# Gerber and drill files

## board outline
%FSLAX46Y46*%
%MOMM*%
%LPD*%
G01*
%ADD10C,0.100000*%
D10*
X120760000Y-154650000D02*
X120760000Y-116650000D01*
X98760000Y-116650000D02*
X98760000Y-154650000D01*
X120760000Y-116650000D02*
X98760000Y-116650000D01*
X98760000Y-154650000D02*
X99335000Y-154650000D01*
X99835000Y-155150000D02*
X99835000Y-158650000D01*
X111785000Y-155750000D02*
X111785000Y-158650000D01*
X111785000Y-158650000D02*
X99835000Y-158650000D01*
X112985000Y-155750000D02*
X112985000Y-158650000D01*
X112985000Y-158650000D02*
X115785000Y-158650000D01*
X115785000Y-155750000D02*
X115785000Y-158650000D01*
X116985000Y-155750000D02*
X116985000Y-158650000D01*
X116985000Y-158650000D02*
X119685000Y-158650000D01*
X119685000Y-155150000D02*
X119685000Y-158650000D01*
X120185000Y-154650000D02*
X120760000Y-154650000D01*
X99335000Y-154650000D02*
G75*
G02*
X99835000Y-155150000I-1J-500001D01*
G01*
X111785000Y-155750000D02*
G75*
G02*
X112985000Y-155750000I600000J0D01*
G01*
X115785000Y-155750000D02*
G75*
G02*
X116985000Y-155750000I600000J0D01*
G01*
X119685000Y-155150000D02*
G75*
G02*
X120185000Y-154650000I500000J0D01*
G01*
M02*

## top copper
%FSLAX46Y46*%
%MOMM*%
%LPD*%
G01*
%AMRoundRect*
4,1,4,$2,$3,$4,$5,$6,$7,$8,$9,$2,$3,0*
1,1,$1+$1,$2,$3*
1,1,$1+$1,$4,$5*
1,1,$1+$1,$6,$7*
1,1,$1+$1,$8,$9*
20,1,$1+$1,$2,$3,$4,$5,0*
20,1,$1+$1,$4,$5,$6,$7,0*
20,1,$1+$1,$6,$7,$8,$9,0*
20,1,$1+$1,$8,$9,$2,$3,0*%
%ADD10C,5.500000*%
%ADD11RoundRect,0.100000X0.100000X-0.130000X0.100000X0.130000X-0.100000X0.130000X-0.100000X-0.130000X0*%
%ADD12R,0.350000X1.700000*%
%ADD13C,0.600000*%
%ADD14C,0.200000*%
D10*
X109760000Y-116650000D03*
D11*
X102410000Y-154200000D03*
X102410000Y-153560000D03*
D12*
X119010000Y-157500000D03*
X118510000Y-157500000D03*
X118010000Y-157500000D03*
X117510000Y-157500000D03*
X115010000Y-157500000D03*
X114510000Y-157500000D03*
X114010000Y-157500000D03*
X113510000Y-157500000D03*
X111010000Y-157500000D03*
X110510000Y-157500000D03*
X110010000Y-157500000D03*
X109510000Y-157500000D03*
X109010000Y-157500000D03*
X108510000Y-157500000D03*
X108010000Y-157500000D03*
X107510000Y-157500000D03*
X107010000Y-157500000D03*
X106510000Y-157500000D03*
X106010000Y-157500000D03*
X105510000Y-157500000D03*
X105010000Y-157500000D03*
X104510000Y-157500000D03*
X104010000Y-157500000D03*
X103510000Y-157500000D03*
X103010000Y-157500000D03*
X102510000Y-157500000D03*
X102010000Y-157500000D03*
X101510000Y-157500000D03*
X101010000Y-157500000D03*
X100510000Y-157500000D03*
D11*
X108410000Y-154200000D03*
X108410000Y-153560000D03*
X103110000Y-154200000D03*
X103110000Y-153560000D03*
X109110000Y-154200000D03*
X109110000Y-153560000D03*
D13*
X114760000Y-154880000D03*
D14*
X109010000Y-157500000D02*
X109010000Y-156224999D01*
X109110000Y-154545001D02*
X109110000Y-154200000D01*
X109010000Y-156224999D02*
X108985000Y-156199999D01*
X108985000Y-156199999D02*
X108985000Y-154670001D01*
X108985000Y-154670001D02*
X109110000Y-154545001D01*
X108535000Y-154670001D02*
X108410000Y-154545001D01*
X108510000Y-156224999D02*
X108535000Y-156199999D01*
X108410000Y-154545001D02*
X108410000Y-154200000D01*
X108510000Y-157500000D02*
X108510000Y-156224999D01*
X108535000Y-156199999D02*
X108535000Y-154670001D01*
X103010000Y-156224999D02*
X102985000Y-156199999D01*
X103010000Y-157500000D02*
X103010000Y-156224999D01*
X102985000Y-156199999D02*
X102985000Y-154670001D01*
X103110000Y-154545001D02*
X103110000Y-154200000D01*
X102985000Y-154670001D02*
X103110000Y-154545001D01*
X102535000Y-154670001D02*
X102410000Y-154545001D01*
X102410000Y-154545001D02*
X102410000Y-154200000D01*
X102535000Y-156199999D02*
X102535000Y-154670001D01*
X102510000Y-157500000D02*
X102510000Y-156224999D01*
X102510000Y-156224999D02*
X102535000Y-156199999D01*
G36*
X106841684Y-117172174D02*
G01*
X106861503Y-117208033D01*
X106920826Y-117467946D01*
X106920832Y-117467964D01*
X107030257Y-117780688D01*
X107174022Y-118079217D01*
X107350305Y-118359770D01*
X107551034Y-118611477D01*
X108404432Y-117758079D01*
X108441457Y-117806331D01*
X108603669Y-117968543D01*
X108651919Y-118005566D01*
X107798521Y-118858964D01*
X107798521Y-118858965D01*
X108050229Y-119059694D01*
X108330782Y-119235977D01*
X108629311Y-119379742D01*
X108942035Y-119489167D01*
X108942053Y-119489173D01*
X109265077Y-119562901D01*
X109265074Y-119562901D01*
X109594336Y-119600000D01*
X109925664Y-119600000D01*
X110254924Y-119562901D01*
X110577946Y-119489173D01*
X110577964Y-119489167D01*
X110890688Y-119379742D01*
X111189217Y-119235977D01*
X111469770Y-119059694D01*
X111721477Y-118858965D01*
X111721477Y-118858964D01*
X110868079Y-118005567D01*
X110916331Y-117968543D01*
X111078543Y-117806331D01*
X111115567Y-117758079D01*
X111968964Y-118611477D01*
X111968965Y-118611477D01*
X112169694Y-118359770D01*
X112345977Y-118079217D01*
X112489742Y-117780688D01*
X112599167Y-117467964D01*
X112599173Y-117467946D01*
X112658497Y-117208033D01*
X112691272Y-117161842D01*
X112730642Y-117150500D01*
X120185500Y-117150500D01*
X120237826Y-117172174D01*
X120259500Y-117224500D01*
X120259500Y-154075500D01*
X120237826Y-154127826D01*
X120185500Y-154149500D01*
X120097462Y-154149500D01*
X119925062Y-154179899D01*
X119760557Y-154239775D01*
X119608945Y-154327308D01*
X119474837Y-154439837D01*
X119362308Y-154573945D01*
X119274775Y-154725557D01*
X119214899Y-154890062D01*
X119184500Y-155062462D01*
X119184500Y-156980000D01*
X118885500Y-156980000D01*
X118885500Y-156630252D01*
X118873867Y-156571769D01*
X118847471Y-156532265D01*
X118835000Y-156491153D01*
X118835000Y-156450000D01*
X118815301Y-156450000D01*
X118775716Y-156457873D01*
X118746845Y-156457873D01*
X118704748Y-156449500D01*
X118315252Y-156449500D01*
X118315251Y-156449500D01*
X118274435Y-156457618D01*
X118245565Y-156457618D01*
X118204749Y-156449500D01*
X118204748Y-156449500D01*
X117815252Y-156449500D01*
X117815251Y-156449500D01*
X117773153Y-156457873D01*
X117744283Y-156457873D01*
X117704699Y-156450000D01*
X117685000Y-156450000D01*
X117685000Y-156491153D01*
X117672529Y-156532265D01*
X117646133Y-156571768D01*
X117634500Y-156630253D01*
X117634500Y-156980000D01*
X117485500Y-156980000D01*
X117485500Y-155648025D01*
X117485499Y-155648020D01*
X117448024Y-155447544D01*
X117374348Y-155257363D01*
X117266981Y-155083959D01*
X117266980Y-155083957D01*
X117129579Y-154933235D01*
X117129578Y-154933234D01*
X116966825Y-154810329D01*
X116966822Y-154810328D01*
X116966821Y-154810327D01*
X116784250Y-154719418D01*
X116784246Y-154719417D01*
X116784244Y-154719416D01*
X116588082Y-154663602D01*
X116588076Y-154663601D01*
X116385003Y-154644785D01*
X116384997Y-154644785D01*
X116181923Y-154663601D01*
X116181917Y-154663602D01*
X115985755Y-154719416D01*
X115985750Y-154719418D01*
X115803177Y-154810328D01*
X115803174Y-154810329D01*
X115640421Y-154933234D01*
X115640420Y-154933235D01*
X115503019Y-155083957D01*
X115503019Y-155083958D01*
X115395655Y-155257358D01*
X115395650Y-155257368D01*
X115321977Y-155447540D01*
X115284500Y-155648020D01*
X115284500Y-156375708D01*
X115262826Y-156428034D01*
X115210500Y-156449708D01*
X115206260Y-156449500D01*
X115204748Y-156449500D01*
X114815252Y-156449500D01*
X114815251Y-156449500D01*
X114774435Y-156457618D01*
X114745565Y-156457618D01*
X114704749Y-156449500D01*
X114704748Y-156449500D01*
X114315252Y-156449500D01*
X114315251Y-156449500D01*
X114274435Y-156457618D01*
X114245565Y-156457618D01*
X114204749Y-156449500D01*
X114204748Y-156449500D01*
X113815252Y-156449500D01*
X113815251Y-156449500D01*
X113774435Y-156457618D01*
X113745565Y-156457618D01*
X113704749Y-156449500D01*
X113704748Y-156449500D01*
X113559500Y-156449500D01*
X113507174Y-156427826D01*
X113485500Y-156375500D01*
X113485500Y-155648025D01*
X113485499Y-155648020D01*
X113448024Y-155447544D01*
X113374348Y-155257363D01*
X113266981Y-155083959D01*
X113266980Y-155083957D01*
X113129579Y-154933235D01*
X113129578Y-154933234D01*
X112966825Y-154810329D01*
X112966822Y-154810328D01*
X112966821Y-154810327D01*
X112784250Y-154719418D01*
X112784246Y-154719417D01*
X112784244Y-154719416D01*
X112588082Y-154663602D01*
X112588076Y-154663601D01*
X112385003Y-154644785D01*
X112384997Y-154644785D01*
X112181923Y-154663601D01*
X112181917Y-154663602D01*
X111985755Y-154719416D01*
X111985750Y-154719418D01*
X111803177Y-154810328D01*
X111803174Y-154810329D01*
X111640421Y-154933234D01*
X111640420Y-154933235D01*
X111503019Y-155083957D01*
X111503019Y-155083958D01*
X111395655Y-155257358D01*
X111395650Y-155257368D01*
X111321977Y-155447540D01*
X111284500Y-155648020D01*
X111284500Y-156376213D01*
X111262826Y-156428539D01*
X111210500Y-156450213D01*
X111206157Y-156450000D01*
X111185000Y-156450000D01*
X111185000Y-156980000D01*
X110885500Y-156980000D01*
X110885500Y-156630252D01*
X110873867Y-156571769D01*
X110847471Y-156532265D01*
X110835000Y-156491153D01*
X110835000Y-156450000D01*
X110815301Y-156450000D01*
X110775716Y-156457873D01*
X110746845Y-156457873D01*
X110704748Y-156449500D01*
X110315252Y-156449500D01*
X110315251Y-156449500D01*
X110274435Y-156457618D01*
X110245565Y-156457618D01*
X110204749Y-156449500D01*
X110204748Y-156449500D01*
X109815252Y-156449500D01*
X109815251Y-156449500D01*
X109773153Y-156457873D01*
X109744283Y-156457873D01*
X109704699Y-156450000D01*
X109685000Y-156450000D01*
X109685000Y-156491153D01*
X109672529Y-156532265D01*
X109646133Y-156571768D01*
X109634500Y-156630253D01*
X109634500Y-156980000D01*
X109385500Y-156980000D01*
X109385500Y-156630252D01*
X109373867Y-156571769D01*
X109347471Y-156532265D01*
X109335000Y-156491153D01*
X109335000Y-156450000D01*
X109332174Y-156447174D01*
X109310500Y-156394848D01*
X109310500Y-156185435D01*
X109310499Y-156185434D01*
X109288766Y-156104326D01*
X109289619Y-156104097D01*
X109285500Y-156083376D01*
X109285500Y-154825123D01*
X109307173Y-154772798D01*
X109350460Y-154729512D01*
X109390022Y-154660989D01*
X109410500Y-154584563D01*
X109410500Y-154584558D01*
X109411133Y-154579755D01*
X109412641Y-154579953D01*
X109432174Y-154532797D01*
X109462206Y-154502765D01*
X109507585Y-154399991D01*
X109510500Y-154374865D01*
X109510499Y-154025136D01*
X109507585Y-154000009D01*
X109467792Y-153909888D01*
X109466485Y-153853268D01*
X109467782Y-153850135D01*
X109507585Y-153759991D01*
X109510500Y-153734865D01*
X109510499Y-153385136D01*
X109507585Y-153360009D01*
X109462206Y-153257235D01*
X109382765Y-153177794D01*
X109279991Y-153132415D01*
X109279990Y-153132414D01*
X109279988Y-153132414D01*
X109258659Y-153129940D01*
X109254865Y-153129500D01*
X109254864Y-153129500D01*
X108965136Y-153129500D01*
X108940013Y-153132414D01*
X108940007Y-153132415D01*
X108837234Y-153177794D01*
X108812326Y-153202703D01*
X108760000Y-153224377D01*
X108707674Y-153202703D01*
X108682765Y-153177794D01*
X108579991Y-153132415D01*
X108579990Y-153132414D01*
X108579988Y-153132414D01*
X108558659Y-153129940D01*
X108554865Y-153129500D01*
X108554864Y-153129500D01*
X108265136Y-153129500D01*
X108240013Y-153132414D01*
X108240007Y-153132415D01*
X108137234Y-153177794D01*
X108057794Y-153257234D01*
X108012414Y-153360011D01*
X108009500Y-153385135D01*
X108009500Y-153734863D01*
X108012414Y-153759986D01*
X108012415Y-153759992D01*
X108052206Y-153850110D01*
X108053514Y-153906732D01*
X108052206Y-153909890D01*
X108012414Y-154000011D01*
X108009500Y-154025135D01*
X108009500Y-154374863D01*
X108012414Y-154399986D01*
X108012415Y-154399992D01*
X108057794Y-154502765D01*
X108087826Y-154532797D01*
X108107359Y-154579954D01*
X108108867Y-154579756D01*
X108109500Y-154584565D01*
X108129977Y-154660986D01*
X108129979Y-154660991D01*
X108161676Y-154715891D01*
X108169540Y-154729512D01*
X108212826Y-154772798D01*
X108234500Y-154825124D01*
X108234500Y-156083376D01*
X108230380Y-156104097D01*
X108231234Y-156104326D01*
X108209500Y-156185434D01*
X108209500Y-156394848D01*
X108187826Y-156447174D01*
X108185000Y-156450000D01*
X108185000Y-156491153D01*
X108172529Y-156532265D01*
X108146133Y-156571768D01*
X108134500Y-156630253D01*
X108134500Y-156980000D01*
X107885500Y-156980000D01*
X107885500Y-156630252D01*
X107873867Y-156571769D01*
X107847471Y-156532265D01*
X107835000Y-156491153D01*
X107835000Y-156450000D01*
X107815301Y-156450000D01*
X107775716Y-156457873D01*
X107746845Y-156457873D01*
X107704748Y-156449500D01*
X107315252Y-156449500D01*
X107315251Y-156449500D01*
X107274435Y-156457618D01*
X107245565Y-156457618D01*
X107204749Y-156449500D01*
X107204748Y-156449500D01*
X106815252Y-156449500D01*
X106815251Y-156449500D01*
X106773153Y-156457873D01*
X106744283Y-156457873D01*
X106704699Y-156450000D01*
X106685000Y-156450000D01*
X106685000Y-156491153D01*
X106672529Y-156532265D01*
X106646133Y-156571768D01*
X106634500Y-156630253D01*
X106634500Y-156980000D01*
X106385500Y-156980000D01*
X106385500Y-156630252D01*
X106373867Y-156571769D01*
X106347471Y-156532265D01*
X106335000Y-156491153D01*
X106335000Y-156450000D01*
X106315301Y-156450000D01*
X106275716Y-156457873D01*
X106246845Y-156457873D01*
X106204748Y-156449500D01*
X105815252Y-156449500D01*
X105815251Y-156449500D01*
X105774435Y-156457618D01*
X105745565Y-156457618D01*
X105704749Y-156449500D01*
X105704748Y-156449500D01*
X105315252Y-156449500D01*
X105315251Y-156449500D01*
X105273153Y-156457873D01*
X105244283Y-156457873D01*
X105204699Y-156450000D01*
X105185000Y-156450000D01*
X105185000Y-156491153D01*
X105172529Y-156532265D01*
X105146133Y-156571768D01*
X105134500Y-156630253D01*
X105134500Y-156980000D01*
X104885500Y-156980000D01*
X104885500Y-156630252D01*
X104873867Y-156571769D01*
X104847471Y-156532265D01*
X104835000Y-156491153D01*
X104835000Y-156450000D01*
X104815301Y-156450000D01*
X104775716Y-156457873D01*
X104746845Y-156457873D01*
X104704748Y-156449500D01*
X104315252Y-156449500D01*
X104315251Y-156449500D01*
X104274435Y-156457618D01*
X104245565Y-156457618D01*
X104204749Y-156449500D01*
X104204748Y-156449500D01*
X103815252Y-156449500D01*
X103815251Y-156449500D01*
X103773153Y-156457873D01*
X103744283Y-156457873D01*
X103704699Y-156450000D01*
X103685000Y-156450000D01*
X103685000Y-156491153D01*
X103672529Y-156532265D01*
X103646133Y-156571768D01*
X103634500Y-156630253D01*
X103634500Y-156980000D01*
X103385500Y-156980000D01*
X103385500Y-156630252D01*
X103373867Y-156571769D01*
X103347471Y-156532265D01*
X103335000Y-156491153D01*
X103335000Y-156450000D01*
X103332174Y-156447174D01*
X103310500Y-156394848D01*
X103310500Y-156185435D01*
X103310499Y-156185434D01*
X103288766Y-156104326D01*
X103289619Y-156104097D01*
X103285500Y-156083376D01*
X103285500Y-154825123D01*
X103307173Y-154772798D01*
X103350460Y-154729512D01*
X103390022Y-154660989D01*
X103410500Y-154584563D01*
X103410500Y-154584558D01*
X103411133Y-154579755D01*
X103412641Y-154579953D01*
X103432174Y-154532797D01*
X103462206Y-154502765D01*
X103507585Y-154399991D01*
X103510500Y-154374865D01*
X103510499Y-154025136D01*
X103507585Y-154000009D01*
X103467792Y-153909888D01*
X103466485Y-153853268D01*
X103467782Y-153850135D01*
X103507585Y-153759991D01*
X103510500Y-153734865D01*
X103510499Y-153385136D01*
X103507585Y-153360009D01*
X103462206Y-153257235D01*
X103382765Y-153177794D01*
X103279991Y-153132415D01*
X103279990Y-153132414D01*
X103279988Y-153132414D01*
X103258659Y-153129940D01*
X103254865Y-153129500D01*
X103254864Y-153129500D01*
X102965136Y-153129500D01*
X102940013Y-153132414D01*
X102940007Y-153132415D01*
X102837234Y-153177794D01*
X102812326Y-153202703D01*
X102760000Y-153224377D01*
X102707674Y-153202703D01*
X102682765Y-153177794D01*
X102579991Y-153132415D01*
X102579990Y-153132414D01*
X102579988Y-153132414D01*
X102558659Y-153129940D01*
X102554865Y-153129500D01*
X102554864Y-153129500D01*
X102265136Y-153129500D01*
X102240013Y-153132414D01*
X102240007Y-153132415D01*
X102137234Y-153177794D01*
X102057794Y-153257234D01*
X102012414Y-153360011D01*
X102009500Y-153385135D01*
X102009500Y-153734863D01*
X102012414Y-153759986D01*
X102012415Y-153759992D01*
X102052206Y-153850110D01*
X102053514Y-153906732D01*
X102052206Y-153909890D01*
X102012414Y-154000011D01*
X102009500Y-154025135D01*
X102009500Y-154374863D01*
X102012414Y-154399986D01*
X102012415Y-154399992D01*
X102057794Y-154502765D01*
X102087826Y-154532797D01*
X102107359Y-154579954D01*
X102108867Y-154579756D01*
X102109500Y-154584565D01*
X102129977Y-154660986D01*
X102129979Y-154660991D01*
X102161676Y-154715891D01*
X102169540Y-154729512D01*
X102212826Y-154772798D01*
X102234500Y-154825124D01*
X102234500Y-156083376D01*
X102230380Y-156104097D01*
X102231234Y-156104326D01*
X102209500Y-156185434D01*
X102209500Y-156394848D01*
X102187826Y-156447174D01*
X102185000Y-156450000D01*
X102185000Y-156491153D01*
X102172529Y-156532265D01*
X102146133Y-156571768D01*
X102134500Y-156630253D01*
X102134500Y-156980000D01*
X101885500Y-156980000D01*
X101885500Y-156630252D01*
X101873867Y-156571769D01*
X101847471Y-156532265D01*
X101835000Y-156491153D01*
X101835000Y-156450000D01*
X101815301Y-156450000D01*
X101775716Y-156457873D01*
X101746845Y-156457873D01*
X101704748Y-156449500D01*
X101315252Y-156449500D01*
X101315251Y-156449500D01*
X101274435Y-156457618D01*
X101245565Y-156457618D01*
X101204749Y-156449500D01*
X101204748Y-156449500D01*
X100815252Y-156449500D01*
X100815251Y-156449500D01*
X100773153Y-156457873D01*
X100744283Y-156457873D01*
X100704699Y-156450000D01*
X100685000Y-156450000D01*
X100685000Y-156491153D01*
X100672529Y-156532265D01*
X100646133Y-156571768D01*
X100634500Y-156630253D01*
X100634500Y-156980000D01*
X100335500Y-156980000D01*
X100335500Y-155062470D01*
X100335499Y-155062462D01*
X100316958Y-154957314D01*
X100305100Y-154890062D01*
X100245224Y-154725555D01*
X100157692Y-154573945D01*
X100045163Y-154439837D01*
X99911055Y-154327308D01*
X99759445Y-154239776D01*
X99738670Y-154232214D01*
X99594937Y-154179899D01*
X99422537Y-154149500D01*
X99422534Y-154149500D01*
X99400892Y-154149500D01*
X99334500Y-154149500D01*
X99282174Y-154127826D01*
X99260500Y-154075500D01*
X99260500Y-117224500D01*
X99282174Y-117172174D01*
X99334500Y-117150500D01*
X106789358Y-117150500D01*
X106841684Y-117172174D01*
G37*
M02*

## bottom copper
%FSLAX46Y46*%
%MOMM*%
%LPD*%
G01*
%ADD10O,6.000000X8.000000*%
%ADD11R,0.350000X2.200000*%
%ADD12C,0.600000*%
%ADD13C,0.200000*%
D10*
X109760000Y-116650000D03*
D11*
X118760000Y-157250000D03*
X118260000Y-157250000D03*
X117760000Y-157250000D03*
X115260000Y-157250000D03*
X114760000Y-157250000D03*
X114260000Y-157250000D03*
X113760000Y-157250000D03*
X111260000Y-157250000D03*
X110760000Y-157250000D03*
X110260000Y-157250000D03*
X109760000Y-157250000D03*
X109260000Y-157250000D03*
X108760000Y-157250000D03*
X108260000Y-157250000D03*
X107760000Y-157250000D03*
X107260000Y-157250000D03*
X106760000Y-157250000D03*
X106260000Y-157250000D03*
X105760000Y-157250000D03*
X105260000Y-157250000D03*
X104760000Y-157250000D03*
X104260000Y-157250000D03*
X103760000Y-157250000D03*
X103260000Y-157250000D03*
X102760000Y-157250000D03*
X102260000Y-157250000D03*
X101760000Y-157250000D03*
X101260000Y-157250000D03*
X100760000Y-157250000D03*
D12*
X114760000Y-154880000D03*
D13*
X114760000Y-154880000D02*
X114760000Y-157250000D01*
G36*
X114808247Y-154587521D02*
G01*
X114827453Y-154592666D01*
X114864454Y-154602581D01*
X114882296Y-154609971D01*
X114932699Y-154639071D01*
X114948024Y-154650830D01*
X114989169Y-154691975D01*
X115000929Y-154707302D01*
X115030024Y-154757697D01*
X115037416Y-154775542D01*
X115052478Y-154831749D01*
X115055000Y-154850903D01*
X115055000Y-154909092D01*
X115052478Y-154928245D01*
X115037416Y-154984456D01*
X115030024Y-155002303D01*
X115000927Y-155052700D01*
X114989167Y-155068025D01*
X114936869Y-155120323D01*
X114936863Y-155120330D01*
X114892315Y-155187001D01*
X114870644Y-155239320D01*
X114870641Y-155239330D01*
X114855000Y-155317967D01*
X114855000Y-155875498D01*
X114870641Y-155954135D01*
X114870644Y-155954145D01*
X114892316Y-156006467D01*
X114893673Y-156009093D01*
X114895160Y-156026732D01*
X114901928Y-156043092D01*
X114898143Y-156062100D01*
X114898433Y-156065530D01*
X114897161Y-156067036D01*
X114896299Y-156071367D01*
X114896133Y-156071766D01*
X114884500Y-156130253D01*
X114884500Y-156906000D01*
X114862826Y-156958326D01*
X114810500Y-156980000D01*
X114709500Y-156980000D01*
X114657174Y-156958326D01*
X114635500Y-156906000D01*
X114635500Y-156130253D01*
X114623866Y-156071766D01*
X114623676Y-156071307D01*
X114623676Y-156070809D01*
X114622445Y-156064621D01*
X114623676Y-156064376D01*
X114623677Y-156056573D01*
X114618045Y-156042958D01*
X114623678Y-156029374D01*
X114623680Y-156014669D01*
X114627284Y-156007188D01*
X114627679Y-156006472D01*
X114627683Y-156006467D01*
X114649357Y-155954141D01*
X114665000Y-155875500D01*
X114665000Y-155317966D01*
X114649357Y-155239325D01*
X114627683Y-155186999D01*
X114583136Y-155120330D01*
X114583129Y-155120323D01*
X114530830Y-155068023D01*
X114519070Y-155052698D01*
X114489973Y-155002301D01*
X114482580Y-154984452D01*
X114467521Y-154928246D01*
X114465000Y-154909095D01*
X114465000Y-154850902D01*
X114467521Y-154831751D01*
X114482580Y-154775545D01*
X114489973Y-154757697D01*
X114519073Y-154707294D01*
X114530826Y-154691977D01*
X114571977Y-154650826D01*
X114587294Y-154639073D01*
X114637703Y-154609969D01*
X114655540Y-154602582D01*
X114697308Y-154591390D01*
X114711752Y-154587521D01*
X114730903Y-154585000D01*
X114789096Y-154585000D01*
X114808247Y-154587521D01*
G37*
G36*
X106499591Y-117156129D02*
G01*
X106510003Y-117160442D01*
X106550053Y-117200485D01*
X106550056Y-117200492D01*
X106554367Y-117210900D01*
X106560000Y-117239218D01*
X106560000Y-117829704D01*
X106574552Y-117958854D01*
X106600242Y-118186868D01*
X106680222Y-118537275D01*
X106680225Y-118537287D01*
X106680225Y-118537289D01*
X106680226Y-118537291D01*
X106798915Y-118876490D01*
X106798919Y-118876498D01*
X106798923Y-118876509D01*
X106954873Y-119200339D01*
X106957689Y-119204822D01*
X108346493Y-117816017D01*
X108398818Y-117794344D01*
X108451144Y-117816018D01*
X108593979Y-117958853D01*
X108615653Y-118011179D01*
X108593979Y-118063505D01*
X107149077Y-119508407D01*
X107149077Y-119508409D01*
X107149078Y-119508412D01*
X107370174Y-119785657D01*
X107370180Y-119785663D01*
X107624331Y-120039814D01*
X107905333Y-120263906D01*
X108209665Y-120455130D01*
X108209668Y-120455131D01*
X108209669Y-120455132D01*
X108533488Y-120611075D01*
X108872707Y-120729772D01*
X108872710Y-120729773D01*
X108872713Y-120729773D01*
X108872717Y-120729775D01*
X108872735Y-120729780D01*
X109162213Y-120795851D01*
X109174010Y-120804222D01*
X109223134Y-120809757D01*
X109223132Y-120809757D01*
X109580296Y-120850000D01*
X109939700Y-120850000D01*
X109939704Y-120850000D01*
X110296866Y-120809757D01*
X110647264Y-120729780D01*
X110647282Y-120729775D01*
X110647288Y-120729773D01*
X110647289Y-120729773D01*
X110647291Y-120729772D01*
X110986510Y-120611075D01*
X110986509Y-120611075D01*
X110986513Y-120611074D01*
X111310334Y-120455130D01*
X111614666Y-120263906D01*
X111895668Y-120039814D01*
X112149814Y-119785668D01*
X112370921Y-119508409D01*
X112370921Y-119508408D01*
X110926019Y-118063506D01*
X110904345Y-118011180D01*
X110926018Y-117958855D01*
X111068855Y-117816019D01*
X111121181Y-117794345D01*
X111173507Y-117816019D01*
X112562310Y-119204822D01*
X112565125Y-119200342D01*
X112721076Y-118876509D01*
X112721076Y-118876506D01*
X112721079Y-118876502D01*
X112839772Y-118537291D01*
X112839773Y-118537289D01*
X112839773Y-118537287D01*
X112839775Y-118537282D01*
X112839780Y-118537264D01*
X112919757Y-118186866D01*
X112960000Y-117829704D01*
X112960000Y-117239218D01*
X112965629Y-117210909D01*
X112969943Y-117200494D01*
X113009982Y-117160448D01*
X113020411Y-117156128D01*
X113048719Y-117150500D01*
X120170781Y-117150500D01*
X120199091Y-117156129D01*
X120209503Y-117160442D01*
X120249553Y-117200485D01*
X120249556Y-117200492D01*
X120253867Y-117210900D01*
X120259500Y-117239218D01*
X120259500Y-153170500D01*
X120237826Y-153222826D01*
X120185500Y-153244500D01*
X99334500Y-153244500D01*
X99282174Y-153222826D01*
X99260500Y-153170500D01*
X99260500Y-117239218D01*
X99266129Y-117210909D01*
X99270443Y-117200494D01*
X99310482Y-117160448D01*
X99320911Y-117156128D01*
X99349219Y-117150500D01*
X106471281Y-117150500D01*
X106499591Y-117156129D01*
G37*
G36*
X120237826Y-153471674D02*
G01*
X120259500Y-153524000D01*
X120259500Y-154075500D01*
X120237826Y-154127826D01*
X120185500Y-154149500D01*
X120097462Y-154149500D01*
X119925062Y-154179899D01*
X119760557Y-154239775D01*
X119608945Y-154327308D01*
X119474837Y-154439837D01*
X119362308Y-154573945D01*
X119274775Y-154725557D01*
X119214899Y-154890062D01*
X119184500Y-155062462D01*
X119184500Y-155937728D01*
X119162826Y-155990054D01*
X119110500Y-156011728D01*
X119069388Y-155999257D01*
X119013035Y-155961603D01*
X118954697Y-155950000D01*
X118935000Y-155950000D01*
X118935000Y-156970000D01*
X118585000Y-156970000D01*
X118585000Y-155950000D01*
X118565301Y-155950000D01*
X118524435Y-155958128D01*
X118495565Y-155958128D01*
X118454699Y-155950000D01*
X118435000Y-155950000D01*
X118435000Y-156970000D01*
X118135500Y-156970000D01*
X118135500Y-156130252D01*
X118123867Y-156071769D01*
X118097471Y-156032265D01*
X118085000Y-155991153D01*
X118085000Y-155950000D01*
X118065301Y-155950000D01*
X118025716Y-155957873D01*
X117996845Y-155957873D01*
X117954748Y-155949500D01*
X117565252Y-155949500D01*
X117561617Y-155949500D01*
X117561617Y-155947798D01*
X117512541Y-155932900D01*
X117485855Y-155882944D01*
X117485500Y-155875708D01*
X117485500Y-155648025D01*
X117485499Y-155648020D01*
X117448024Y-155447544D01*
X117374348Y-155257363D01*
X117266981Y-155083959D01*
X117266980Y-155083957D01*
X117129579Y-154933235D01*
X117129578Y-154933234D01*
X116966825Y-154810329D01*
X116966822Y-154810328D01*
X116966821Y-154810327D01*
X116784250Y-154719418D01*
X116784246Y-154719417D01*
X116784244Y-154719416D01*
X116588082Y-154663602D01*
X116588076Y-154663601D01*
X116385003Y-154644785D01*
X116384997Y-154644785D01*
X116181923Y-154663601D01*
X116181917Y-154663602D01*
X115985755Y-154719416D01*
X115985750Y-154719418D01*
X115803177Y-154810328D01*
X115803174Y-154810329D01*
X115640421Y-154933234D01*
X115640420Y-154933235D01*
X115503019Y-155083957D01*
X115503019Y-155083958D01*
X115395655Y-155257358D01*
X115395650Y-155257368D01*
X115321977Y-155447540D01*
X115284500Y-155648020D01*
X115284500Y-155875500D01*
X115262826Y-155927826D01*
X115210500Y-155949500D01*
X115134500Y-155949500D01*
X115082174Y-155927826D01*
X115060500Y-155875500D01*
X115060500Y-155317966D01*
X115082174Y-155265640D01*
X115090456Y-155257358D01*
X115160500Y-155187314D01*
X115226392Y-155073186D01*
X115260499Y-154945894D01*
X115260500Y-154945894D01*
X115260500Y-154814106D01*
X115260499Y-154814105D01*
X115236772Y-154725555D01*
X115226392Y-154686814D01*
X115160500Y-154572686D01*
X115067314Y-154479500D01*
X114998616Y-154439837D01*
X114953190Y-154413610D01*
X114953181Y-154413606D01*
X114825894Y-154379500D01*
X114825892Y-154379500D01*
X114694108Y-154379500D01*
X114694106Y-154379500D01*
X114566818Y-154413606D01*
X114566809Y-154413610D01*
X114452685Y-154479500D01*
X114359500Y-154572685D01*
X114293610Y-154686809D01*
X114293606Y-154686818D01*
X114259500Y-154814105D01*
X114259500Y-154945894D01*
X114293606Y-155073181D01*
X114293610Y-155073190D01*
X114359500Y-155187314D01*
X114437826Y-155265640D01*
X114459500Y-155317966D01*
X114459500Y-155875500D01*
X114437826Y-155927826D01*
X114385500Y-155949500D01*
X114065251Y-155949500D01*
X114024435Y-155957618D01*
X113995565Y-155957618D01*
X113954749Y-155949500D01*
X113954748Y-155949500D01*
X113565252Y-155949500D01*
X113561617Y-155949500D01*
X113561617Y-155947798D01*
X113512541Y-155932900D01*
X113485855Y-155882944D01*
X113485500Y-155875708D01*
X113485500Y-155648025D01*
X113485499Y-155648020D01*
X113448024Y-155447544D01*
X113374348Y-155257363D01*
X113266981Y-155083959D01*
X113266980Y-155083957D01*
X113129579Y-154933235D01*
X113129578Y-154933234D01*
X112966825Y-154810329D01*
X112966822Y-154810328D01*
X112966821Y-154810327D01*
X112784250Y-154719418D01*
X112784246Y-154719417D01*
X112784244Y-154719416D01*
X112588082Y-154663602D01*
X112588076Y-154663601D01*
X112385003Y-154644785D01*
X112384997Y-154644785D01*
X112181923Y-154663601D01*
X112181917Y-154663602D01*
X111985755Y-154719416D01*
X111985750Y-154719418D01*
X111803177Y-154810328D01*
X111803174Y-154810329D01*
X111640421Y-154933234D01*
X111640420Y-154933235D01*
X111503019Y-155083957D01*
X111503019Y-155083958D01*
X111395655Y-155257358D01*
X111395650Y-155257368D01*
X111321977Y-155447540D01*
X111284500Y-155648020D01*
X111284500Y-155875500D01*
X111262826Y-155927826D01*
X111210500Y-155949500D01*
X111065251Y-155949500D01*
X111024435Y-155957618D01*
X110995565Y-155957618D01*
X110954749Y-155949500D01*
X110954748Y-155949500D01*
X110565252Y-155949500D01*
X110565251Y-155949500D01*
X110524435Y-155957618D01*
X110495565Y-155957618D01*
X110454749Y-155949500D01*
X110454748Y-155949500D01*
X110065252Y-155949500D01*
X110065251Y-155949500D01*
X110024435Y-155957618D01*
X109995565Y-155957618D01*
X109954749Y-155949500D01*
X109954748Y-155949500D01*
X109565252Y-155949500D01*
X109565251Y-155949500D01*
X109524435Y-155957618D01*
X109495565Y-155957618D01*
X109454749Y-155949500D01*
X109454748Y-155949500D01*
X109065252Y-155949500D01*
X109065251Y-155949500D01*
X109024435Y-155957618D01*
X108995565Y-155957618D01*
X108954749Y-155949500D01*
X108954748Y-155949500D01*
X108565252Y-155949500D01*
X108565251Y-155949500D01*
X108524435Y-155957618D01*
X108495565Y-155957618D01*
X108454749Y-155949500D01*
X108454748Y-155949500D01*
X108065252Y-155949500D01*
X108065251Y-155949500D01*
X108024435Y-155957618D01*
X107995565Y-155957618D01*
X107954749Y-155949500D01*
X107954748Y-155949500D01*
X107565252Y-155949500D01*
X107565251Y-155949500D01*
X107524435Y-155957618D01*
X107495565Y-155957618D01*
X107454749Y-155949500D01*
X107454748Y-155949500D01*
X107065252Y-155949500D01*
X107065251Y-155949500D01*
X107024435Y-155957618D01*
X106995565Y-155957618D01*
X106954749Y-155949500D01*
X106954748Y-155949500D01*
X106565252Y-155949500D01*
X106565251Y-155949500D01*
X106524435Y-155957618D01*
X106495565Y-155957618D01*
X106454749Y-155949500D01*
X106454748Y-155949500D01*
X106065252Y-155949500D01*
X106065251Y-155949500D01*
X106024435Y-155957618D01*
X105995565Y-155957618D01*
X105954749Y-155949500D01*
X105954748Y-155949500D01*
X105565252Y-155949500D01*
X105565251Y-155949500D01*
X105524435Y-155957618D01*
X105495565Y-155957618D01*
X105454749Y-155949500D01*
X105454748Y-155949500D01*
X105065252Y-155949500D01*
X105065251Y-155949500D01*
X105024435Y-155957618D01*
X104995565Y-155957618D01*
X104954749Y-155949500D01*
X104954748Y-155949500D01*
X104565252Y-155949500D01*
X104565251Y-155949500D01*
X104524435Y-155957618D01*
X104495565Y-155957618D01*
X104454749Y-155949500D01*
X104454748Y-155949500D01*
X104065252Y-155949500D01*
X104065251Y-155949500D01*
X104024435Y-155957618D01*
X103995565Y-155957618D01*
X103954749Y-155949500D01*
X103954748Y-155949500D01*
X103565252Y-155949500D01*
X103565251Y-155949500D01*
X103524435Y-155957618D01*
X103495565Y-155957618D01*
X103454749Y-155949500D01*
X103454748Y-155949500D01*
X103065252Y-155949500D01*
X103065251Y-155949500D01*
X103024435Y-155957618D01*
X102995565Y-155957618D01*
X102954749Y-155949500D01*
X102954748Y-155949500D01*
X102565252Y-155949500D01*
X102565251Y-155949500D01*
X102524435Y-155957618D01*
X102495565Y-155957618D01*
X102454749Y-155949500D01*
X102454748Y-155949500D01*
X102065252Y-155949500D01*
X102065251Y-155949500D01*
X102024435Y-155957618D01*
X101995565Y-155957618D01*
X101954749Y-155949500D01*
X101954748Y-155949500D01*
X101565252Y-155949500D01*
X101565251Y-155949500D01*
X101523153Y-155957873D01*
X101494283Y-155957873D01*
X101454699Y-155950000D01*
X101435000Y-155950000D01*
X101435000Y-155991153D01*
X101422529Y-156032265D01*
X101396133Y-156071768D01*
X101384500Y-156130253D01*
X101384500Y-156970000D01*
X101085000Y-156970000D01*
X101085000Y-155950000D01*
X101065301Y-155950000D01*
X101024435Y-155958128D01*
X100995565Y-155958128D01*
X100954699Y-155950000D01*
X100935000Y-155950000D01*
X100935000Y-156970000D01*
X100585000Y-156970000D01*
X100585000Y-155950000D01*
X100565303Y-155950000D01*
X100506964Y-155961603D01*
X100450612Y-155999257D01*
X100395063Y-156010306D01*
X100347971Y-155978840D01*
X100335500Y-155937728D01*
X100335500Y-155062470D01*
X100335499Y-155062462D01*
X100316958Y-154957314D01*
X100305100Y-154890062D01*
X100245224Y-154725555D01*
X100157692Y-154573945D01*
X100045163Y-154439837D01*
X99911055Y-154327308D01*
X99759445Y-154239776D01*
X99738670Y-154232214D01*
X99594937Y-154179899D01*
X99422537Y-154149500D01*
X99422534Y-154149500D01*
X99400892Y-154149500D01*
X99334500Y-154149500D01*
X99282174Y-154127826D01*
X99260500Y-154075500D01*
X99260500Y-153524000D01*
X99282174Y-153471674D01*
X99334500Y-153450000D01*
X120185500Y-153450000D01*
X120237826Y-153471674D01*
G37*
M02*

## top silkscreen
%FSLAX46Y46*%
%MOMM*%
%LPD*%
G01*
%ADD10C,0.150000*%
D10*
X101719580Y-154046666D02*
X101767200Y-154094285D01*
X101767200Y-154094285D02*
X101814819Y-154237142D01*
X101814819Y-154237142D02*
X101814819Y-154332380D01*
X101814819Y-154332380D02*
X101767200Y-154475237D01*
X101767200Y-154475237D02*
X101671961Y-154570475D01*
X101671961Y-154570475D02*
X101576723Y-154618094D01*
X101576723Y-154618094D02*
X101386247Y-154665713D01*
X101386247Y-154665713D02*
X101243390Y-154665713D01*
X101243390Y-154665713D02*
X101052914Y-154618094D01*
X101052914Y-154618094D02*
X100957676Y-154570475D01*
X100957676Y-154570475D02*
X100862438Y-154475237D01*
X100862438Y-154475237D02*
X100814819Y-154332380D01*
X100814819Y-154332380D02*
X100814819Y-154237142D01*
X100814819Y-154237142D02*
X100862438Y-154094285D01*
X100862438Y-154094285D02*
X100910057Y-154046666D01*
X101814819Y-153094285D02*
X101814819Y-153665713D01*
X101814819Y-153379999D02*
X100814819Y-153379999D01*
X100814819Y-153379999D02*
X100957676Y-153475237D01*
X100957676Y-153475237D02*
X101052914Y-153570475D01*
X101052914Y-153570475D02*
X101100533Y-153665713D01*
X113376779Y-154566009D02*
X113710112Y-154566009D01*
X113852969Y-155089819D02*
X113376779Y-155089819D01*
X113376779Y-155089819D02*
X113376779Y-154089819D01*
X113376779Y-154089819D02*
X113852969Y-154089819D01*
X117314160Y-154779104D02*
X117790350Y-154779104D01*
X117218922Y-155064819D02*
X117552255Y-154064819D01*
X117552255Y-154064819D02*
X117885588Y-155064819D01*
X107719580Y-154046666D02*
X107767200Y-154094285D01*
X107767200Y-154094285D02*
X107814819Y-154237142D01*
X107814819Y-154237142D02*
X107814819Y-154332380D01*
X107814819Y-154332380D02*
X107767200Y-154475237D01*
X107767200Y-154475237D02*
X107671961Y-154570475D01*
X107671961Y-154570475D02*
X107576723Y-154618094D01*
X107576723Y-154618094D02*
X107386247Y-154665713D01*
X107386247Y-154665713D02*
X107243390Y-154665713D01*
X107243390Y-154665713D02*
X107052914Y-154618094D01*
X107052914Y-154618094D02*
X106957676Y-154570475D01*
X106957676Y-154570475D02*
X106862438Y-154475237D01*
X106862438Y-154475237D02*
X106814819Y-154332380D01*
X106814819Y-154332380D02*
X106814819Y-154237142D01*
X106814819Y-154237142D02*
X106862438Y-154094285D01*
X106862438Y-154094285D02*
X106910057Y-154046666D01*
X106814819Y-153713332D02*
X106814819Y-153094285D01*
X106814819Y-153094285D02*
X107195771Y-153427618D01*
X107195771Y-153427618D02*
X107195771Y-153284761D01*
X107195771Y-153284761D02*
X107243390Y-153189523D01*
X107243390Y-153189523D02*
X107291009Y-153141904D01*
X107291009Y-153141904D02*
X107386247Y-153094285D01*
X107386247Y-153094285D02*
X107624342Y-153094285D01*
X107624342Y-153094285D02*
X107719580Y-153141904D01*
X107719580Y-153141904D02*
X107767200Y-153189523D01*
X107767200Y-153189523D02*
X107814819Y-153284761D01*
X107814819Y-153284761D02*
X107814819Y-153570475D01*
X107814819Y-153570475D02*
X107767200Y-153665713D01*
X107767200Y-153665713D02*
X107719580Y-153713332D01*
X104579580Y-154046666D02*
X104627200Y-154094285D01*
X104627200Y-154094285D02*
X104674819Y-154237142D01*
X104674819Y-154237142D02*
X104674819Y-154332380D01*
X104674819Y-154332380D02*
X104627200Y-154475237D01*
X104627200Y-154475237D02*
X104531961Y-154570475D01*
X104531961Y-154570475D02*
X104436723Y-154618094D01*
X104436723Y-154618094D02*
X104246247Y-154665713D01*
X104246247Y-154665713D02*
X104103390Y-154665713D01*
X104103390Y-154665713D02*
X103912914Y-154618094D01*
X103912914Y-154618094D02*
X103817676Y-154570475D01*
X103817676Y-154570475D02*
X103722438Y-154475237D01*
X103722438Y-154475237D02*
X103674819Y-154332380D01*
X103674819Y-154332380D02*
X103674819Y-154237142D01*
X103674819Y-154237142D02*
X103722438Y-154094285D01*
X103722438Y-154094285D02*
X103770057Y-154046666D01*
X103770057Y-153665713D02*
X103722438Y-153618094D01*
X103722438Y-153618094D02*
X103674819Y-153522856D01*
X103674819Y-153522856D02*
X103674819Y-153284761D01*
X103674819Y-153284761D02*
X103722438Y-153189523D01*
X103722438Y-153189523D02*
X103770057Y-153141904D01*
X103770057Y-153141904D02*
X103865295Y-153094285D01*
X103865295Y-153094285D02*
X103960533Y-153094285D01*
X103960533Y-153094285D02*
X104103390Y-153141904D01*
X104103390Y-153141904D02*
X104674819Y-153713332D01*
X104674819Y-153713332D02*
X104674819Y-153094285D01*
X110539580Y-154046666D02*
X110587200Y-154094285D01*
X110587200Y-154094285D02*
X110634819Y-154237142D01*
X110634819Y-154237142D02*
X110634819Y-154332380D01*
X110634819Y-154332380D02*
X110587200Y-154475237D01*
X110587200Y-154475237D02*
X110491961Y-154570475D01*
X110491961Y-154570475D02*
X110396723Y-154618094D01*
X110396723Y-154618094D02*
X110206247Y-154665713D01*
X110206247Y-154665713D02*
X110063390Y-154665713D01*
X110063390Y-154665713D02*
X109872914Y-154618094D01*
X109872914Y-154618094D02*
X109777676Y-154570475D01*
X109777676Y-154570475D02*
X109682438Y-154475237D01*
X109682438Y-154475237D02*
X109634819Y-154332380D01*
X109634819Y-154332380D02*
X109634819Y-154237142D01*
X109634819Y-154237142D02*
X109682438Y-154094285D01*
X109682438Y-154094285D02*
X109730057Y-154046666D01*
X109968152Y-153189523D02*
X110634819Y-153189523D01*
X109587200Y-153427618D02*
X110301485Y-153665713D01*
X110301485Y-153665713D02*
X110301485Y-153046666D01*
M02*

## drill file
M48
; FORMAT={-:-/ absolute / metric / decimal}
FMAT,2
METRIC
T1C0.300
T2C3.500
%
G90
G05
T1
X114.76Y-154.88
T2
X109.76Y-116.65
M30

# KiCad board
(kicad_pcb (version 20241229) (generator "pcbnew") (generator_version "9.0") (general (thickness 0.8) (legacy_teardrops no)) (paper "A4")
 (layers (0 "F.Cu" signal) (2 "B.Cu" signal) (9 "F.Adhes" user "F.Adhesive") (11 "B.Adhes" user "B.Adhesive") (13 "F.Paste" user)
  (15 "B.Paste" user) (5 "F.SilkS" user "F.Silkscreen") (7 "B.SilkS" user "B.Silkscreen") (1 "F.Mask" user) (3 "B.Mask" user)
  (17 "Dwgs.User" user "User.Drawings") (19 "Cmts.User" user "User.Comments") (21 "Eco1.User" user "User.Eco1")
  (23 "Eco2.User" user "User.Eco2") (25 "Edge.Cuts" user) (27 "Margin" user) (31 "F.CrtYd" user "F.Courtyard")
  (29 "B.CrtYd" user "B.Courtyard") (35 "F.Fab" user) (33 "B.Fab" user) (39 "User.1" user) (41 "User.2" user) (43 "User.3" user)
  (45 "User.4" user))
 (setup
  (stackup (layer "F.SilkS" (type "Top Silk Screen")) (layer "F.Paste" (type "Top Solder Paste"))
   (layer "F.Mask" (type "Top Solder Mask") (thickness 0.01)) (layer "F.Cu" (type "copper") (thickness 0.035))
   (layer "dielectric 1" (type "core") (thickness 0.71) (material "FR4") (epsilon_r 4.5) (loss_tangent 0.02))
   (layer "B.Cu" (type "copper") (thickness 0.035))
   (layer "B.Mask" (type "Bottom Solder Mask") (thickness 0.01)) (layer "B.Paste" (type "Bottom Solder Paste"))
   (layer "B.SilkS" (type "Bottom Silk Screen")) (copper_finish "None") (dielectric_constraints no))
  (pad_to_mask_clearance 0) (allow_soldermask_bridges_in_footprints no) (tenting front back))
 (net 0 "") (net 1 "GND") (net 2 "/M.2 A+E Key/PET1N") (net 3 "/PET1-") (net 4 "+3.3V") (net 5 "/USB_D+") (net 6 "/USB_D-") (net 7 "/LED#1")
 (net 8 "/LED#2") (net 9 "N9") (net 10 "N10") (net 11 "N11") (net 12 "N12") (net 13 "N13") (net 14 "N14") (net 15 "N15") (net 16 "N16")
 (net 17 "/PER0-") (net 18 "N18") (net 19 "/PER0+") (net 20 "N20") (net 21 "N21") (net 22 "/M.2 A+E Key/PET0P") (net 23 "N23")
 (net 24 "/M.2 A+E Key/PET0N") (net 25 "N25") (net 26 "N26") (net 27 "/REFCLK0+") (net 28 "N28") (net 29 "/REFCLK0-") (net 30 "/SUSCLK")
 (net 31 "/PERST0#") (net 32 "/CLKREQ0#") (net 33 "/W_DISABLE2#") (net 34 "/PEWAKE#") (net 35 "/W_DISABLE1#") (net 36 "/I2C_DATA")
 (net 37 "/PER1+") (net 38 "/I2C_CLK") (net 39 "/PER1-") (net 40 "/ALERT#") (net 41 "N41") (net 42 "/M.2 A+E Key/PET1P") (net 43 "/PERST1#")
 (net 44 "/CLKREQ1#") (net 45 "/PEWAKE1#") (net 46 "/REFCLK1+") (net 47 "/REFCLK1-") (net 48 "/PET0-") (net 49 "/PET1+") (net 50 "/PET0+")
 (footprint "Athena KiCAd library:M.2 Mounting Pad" (layer "F.Cu") (at 109.76 116.65)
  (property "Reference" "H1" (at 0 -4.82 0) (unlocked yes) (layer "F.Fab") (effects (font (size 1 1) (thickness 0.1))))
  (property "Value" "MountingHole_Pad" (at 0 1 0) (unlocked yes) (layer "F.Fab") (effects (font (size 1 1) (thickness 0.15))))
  (pad "1" thru_hole circle (at 0 0) (size 5.5 5.5) (drill 3.5) (layers "*.Cu" "*.Mask") (remove_unused_layers no) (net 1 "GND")
   (padstack (mode front_inner_back)
    (layer "Inner" (shape circle) (size 5.5 5.5) (zone_connect -1))
    (layer "B.Cu" (shape oval) (size 6 8) (thermal_bridge_angle 45) (zone_connect -1)))))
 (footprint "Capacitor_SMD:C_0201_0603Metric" (layer "F.Cu") (at 102.41 153.88 90)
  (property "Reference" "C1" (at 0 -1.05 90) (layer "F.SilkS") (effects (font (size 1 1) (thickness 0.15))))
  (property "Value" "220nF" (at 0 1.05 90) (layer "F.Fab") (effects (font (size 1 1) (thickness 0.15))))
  (pad "" smd roundrect (at -0.345 0 90) (size 0.318 0.36) (layers "F.Paste") (roundrect_rratio 0.25))
  (pad "" smd roundrect (at 0.345 0 90) (size 0.318 0.36) (layers "F.Paste") (roundrect_rratio 0.25))
  (pad "1" smd roundrect (at -0.32 0 90) (size 0.46 0.4) (layers "F.Cu" "F.Mask") (roundrect_rratio 0.25) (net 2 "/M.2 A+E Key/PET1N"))
  (pad "2" smd roundrect (at 0.32 0 90) (size 0.46 0.4) (layers "F.Cu" "F.Mask") (roundrect_rratio 0.25) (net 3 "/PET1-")))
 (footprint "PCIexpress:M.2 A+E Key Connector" (layer "F.Cu") (at 109.76 157.54)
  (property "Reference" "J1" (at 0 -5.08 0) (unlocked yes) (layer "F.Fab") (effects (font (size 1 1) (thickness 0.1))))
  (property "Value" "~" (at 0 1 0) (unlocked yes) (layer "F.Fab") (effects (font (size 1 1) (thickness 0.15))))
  (fp_line (start -11 -2.89) (end -10.425 -2.89) (stroke (width 0.1) (type default)) (layer "Edge.Cuts"))
  (fp_line (start -9.925 -2.39) (end -9.925 1.11) (stroke (width 0.1) (type default)) (layer "Edge.Cuts"))
  (fp_line (start 2.025 -1.79) (end 2.025 1.11) (stroke (width 0.1) (type default)) (layer "Edge.Cuts"))
  (fp_line (start 2.025 1.11) (end -9.925 1.11) (stroke (width 0.1) (type default)) (layer "Edge.Cuts"))
  (fp_line (start 3.225 -1.79) (end 3.225 1.11) (stroke (width 0.1) (type default)) (layer "Edge.Cuts"))
  (fp_line (start 3.225 1.11) (end 6.025 1.11) (stroke (width 0.1) (type default)) (layer "Edge.Cuts"))
  (fp_line (start 6.025 -1.79) (end 6.025 1.11) (stroke (width 0.1) (type default)) (layer "Edge.Cuts"))
  (fp_line (start 7.225 -1.79) (end 7.225 1.11) (stroke (width 0.1) (type default)) (layer "Edge.Cuts"))
  (fp_line (start 7.225 1.11) (end 9.925 1.11) (stroke (width 0.1) (type default)) (layer "Edge.Cuts"))
  (fp_line (start 9.925 -2.39) (end 9.925 1.11) (stroke (width 0.1) (type default)) (layer "Edge.Cuts"))
  (fp_line (start 10.425 -2.89) (end 11 -2.89) (stroke (width 0.1) (type default)) (layer "Edge.Cuts"))
  (fp_arc (start -10.425 -2.89) (mid -10.071447 -2.743553) (end -9.925 -2.39) (stroke (width 0.1) (type default)) (layer "Edge.Cuts"))
  (fp_arc (start 2.025 -1.79) (mid 2.625 -2.39) (end 3.225 -1.79) (stroke (width 0.1) (type default)) (layer "Edge.Cuts"))
  (fp_arc (start 6.025 -1.79) (mid 6.625 -2.39) (end 7.225 -1.79) (stroke (width 0.1) (type default)) (layer "Edge.Cuts"))
  (fp_arc (start 9.925 -2.39) (mid 10.071447 -2.743553) (end 10.425 -2.89) (stroke (width 0.1) (type default)) (layer "Edge.Cuts"))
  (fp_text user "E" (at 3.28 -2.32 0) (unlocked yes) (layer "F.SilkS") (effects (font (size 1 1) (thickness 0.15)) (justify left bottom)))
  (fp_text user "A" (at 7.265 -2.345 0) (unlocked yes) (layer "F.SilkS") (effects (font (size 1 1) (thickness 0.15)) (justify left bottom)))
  (pad "1" smd rect (at 9.25 -0.04 180) (size 0.35 1.7) (layers "F.Cu") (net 1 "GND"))
  (pad "2" smd rect (at 9 -0.29 180) (size 0.35 2.2) (layers "B.Cu") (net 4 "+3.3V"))
  (pad "3" smd rect (at 8.75 -0.04 180) (size 0.35 1.7) (layers "F.Cu") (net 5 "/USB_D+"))
  (pad "4" smd rect (at 8.5 -0.29 180) (size 0.35 2.2) (layers "B.Cu") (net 4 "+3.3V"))
  (pad "5" smd rect (at 8.25 -0.04 180) (size 0.35 1.7) (layers "F.Cu") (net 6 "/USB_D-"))
  (pad "6" smd rect (at 8 -0.29 180) (size 0.35 2.2) (layers "B.Cu") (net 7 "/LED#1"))
  (pad "7" smd rect (at 7.75 -0.04 180) (size 0.35 1.7) (layers "F.Cu") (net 1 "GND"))
  (pad "16" smd rect (at 5.5 -0.29 180) (size 0.35 2.2) (layers "B.Cu") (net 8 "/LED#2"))
  (pad "17" smd rect (at 5.25 -0.04 180) (size 0.35 1.7) (layers "F.Cu") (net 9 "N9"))
  (pad "18" smd rect (at 5 -0.29 180) (size 0.35 2.2) (layers "B.Cu") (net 1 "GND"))
  (pad "19" smd rect (at 4.75 -0.04 180) (size 0.35 1.7) (layers "F.Cu") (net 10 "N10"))
  (pad "20" smd rect (at 4.5 -0.29 180) (size 0.35 2.2) (layers "B.Cu") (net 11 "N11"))
  (pad "21" smd rect (at 4.25 -0.04 180) (size 0.35 1.7) (layers "F.Cu") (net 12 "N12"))
  (pad "22" smd rect (at 4 -0.29 180) (size 0.35 2.2) (layers "B.Cu") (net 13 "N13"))
  (pad "23" smd rect (at 3.75 -0.04 180) (size 0.35 1.7) (layers "F.Cu") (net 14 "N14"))
  (pad "32" smd rect (at 1.5 -0.29 180) (size 0.35 2.2) (layers "B.Cu") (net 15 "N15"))
  (pad "33" smd rect (at 1.25 -0.04 180) (size 0.35 1.7) (layers "F.Cu") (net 1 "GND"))
  (pad "34" smd rect (at 1 -0.29 180) (size 0.35 2.2) (layers "B.Cu") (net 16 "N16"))
  (pad "35" smd rect (at 0.75 -0.04 180) (size 0.35 1.7) (layers "F.Cu") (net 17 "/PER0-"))
  (pad "36" smd rect (at 0.5 -0.29 180) (size 0.35 2.2) (layers "B.Cu") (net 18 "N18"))
  (pad "37" smd rect (at 0.25 -0.04 180) (size 0.35 1.7) (layers "F.Cu") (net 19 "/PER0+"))
  (pad "38" smd rect (at 0 -0.29 180) (size 0.35 2.2) (layers "B.Cu") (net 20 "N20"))
  (pad "39" smd rect (at -0.25 -0.04 180) (size 0.35 1.7) (layers "F.Cu") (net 1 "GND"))
  (pad "40" smd rect (at -0.5 -0.29 180) (size 0.35 2.2) (layers "B.Cu") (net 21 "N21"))
  (pad "41" smd rect (at -0.75 -0.04 180) (size 0.35 1.7) (layers "F.Cu") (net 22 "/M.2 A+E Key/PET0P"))
  (pad "42" smd rect (at -1 -0.29 180) (size 0.35 2.2) (layers "B.Cu") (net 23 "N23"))
  (pad "43" smd rect (at -1.25 -0.04 180) (size 0.35 1.7) (layers "F.Cu") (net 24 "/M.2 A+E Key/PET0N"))
  (pad "44" smd rect (at -1.5 -0.29 180) (size 0.35 2.2) (layers "B.Cu") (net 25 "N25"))
  (pad "45" smd rect (at -1.75 -0.04 180) (size 0.35 1.7) (layers "F.Cu") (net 1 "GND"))
  (pad "46" smd rect (at -2 -0.29 180) (size 0.35 2.2) (layers "B.Cu") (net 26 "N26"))
  (pad "47" smd rect (at -2.25 -0.04 180) (size 0.35 1.7) (layers "F.Cu") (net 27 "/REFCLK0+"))
  (pad "48" smd rect (at -2.5 -0.29 180) (size 0.35 2.2) (layers "B.Cu") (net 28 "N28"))
  (pad "49" smd rect (at -2.75 -0.04 180) (size 0.35 1.7) (layers "F.Cu") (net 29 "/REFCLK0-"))
  (pad "50" smd rect (at -3 -0.29 180) (size 0.35 2.2) (layers "B.Cu") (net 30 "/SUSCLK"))
  (pad "51" smd rect (at -3.25 -0.04 180) (size 0.35 1.7) (layers "F.Cu") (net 1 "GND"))
  (pad "52" smd rect (at -3.5 -0.29 180) (size 0.35 2.2) (layers "B.Cu") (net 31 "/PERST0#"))
  (pad "53" smd rect (at -3.75 -0.04 180) (size 0.35 1.7) (layers "F.Cu") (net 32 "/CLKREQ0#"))
  (pad "54" smd rect (at -4 -0.29 180) (size 0.35 2.2) (layers "B.Cu") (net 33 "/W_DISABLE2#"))
  (pad "55" smd rect (at -4.25 -0.04 180) (size 0.35 1.7) (layers "F.Cu") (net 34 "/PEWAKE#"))
  (pad "56" smd rect (at -4.5 -0.29 180) (size 0.35 2.2) (layers "B.Cu") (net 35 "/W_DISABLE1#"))
  (pad "57" smd rect (at -4.75 -0.04 180) (size 0.35 1.7) (layers "F.Cu") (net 1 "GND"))
  (pad "58" smd rect (at -5 -0.29 180) (size 0.35 2.2) (layers "B.Cu") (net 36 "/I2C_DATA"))
  (pad "59" smd rect (at -5.25 -0.04 180) (size 0.35 1.7) (layers "F.Cu") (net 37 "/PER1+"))
  (pad "60" smd rect (at -5.5 -0.29 180) (size 0.35 2.2) (layers "B.Cu") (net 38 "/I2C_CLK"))
  (pad "61" smd rect (at -5.75 -0.04 180) (size 0.35 1.7) (layers "F.Cu") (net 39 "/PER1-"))
  (pad "62" smd rect (at -6 -0.29 180) (size 0.35 2.2) (layers "B.Cu") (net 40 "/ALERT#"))
  (pad "63" smd rect (at -6.25 -0.04 180) (size 0.35 1.7) (layers "F.Cu") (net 1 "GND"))
  (pad "64" smd rect (at -6.5 -0.29 180) (size 0.35 2.2) (layers "B.Cu") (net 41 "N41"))
  (pad "65" smd rect (at -6.75 -0.04 180) (size 0.35 1.7) (layers "F.Cu") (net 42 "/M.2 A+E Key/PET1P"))
  (pad "66" smd rect (at -7 -0.29 180) (size 0.35 2.2) (layers "B.Cu") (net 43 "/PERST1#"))
  (pad "67" smd rect (at -7.25 -0.04 180) (size 0.35 1.7) (layers "F.Cu") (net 2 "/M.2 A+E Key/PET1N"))
  (pad "68" smd rect (at -7.5 -0.29 180) (size 0.35 2.2) (layers "B.Cu") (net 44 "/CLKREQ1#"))
  (pad "69" smd rect (at -7.75 -0.04 180) (size 0.35 1.7) (layers "F.Cu") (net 1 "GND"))
  (pad "70" smd rect (at -8 -0.29 180) (size 0.35 2.2) (layers "B.Cu") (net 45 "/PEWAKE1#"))
  (pad "71" smd rect (at -8.25 -0.04 180) (size 0.35 1.7) (layers "F.Cu") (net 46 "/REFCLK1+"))
  (pad "72" smd rect (at -8.5 -0.29 180) (size 0.35 2.2) (layers "B.Cu") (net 4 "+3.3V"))
  (pad "73" smd rect (at -8.75 -0.04 180) (size 0.35 1.7) (layers "F.Cu") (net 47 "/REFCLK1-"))
  (pad "74" smd rect (at -9 -0.29 180) (size 0.35 2.2) (layers "B.Cu") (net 4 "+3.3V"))
  (pad "75" smd rect (at -9.25 -0.04 180) (size 0.35 1.7) (layers "F.Cu") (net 1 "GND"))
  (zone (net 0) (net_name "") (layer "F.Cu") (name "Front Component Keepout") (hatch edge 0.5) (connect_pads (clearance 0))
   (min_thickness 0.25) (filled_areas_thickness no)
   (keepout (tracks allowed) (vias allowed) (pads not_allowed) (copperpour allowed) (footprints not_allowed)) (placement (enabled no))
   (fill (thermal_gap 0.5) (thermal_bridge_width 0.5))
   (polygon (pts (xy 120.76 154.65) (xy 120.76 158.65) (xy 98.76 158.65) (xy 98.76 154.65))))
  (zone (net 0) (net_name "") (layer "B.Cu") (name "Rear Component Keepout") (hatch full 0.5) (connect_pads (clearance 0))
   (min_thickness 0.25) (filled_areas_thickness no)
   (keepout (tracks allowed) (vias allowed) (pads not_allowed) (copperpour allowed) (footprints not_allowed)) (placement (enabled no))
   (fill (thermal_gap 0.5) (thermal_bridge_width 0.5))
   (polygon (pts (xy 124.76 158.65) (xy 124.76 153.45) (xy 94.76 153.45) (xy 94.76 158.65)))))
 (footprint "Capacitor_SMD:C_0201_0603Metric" (layer "F.Cu") (at 108.41 153.88 90)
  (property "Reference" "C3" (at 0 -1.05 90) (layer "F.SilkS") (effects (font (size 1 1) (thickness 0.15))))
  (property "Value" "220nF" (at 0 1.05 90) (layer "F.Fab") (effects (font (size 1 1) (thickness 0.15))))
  (pad "" smd roundrect (at -0.345 0 90) (size 0.318 0.36) (layers "F.Paste") (roundrect_rratio 0.25))
  (pad "" smd roundrect (at 0.345 0 90) (size 0.318 0.36) (layers "F.Paste") (roundrect_rratio 0.25))
  (pad "1" smd roundrect (at -0.32 0 90) (size 0.46 0.4) (layers "F.Cu" "F.Mask") (roundrect_rratio 0.25) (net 24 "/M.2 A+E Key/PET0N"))
  (pad "2" smd roundrect (at 0.32 0 90) (size 0.46 0.4) (layers "F.Cu" "F.Mask") (roundrect_rratio 0.25) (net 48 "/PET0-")))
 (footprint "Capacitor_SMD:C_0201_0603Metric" (layer "F.Cu") (at 103.11 153.88 90)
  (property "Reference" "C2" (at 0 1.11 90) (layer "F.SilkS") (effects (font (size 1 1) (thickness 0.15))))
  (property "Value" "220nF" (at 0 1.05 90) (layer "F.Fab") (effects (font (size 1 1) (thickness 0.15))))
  (pad "" smd roundrect (at -0.345 0 90) (size 0.318 0.36) (layers "F.Paste") (roundrect_rratio 0.25))
  (pad "" smd roundrect (at 0.345 0 90) (size 0.318 0.36) (layers "F.Paste") (roundrect_rratio 0.25))
  (pad "1" smd roundrect (at -0.32 0 90) (size 0.46 0.4) (layers "F.Cu" "F.Mask") (roundrect_rratio 0.25) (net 42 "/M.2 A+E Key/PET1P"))
  (pad "2" smd roundrect (at 0.32 0 90) (size 0.46 0.4) (layers "F.Cu" "F.Mask") (roundrect_rratio 0.25) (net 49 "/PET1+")))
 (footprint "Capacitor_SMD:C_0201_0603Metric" (layer "F.Cu") (at 109.11 153.88 90)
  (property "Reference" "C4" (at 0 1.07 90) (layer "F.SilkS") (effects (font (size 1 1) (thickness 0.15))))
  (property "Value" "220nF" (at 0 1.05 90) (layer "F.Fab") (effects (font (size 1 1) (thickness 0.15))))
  (pad "" smd roundrect (at -0.345 0 90) (size 0.318 0.36) (layers "F.Paste") (roundrect_rratio 0.25))
  (pad "" smd roundrect (at 0.345 0 90) (size 0.318 0.36) (layers "F.Paste") (roundrect_rratio 0.25))
  (pad "1" smd roundrect (at -0.32 0 90) (size 0.46 0.4) (layers "F.Cu" "F.Mask") (roundrect_rratio 0.25) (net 22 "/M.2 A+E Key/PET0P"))
  (pad "2" smd roundrect (at 0.32 0 90) (size 0.46 0.4) (layers "F.Cu" "F.Mask") (roundrect_rratio 0.25) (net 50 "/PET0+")))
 (gr_line (start 120.76 154.65) (end 120.76 116.65) (stroke (width 0.1) (type default)) (layer "Edge.Cuts"))
 (gr_line (start 98.76 116.65) (end 98.76 154.65) (stroke (width 0.1) (type default)) (layer "Edge.Cuts"))
 (gr_line (start 120.76 116.65) (end 98.76 116.65) (stroke (width 0.1) (type default)) (layer "Edge.Cuts"))
 (segment (start 109.01 157.5) (end 109.01 156.224999) (width 0.2) (layer "F.Cu") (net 22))
 (segment (start 109.11 154.545001) (end 109.11 154.2) (width 0.2) (layer "F.Cu") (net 22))
 (segment (start 109.01 156.224999) (end 108.985 156.199999) (width 0.2) (layer "F.Cu") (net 22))
 (segment (start 108.985 156.199999) (end 108.985 154.670001) (width 0.2) (layer "F.Cu") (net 22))
 (segment (start 108.985 154.670001) (end 109.11 154.545001) (width 0.2) (layer "F.Cu") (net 22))
 (segment (start 108.535 154.670001) (end 108.41 154.545001) (width 0.2) (layer "F.Cu") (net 24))
 (segment (start 108.51 156.224999) (end 108.535 156.199999) (width 0.2) (layer "F.Cu") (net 24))
 (segment (start 108.41 154.545001) (end 108.41 154.2) (width 0.2) (layer "F.Cu") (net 24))
 (segment (start 108.51 157.5) (end 108.51 156.224999) (width 0.2) (layer "F.Cu") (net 24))
 (segment (start 108.535 156.199999) (end 108.535 154.670001) (width 0.2) (layer "F.Cu") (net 24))
 (via (at 114.76 154.88) (size 0.6) (drill 0.3) (layers "F.Cu" "B.Cu") (free yes) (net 1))
 (segment (start 114.76 154.88) (end 114.76 157.25) (width 0.2) (layer "B.Cu") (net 1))
 (segment (start 103.01 156.224999) (end 102.985 156.199999) (width 0.2) (layer "F.Cu") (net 42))
 (segment (start 103.01 157.5) (end 103.01 156.224999) (width 0.2) (layer "F.Cu") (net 42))
 (segment (start 102.985 156.199999) (end 102.985 154.670001) (width 0.2) (layer "F.Cu") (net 42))
 (segment (start 103.11 154.545001) (end 103.11 154.2) (width 0.2) (layer "F.Cu") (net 42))
 (segment (start 102.985 154.670001) (end 103.11 154.545001) (width 0.2) (layer "F.Cu") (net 42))
 (segment (start 102.535 154.670001) (end 102.41 154.545001) (width 0.2) (layer "F.Cu") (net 2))
 (segment (start 102.41 154.545001) (end 102.41 154.2) (width 0.2) (layer "F.Cu") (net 2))
 (segment (start 102.535 156.199999) (end 102.535 154.670001) (width 0.2) (layer "F.Cu") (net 2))
 (segment (start 102.51 157.5) (end 102.51 156.224999) (width 0.2) (layer "F.Cu") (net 2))
 (segment (start 102.51 156.224999) (end 102.535 156.199999) (width 0.2) (layer "F.Cu") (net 2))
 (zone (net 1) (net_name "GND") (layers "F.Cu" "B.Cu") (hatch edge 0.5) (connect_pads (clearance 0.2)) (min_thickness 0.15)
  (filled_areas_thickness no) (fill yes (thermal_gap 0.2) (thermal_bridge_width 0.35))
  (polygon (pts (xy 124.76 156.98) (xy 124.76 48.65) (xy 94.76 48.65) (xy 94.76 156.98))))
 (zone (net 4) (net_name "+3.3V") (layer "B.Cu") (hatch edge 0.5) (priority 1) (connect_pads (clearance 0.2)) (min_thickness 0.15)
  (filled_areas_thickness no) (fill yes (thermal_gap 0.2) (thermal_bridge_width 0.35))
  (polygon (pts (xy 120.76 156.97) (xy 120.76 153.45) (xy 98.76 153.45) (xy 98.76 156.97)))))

